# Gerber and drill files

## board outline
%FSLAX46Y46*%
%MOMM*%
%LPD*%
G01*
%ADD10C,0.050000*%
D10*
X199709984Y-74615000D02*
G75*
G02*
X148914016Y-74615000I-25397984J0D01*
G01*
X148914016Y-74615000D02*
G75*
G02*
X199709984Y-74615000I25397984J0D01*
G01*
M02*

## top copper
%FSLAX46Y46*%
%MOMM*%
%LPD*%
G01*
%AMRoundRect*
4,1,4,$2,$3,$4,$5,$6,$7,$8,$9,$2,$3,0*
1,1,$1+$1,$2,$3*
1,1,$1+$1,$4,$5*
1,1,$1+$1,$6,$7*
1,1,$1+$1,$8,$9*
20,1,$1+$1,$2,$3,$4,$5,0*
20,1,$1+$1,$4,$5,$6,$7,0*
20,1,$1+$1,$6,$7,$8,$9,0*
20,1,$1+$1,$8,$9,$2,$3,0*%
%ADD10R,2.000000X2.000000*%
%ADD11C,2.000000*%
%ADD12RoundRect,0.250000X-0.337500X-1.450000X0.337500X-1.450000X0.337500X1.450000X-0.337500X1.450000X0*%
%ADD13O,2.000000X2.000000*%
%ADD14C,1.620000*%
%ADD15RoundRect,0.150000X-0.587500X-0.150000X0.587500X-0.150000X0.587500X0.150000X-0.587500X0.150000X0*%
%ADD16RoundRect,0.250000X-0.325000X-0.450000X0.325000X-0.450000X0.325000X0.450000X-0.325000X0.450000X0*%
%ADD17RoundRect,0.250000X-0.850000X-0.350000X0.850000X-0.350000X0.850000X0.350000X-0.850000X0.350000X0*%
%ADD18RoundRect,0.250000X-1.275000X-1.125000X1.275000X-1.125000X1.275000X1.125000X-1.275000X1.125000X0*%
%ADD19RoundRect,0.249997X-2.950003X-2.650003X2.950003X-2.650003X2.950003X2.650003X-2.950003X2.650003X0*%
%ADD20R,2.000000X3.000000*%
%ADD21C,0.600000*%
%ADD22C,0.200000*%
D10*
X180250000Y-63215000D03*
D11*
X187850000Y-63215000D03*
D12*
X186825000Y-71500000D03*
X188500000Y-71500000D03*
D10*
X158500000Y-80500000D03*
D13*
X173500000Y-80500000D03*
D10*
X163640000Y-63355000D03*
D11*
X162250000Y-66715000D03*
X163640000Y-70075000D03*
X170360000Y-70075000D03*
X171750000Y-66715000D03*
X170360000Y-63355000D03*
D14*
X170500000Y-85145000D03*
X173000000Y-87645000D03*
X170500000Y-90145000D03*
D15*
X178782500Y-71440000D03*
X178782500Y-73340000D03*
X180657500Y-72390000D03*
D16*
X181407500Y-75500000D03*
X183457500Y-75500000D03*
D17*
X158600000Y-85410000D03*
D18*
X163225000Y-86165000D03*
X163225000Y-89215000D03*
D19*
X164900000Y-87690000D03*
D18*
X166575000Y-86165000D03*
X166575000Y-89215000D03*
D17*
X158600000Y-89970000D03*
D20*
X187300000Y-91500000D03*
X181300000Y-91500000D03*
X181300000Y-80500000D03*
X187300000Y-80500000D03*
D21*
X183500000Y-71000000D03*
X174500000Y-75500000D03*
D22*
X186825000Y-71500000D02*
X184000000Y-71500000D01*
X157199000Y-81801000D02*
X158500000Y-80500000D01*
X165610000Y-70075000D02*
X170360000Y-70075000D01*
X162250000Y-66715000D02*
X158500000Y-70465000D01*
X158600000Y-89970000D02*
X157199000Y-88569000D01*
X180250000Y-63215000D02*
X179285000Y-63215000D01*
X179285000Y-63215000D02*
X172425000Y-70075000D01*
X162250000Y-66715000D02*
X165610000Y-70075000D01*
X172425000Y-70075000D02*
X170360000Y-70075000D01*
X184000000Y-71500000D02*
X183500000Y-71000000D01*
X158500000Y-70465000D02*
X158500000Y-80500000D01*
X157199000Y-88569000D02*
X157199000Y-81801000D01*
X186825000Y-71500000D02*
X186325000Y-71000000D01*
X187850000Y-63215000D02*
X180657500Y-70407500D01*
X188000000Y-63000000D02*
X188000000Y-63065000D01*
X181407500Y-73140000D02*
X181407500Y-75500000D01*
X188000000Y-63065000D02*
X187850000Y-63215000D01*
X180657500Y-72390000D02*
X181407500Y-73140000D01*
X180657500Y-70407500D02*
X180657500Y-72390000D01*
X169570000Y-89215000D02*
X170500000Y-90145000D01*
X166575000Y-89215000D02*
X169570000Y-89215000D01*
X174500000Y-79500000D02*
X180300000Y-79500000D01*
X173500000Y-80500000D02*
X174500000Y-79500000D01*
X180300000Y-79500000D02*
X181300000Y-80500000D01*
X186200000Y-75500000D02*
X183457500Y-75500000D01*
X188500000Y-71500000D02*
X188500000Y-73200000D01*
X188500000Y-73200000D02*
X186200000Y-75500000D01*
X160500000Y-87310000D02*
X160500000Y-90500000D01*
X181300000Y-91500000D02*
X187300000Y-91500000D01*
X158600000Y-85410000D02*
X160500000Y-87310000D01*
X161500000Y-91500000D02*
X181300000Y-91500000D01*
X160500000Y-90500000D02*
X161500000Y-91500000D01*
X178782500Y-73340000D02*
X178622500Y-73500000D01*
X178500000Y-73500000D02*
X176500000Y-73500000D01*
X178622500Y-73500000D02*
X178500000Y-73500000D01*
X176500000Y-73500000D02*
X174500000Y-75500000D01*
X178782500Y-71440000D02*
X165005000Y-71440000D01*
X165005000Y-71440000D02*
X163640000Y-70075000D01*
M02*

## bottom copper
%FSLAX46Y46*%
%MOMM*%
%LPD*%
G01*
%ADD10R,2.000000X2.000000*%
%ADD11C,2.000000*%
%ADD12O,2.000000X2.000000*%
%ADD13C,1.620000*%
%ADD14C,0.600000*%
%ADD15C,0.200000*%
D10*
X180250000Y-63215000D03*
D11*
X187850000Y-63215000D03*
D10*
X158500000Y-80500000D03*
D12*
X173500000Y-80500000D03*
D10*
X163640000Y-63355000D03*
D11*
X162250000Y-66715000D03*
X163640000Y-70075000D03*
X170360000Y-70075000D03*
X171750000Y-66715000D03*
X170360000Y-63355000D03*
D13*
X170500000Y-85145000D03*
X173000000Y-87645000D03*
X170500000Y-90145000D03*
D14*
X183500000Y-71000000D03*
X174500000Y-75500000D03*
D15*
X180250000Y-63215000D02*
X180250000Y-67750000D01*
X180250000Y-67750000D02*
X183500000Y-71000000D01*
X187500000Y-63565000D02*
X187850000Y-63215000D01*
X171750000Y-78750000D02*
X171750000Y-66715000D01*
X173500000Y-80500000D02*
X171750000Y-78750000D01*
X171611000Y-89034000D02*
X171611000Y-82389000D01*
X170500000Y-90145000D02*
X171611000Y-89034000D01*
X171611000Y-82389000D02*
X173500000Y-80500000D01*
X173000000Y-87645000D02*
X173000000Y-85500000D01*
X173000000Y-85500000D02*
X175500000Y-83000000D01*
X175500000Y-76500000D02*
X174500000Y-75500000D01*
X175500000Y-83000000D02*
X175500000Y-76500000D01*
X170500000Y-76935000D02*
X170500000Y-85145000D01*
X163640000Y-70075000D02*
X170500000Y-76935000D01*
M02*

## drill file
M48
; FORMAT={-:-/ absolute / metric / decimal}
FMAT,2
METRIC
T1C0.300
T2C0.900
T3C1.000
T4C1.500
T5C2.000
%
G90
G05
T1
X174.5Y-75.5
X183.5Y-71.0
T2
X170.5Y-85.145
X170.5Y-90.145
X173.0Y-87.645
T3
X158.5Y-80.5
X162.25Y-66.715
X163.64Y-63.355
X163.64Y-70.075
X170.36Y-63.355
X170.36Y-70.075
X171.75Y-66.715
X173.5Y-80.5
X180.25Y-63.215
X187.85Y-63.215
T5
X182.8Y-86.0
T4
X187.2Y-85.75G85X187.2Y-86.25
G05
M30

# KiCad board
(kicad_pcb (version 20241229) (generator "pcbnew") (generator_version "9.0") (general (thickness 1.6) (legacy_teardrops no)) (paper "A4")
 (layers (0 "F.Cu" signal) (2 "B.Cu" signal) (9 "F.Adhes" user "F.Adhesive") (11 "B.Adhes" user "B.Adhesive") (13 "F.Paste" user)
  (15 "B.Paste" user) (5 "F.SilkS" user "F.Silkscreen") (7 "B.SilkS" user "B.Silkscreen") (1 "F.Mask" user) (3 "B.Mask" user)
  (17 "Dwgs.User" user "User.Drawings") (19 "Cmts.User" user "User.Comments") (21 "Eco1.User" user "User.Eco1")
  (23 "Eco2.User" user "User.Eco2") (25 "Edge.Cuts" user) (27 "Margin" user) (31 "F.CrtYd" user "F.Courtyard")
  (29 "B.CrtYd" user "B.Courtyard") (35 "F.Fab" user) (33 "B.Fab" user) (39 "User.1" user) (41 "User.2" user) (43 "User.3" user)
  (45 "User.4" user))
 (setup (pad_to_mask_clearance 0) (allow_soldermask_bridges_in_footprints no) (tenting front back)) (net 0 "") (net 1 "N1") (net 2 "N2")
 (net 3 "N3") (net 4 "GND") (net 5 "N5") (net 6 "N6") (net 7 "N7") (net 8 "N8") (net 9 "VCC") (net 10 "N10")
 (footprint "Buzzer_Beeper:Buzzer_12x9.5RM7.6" (layer "F.Cu") (at 180.25 63.215)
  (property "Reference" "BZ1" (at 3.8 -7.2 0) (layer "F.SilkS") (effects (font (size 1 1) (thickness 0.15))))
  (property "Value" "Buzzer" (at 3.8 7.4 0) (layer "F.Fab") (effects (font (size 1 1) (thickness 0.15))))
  (pad "1" thru_hole rect (at 0 0) (size 2 2) (drill 1) (layers "*.Cu" "*.Mask") (remove_unused_layers no) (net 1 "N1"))
  (pad "2" thru_hole circle (at 7.6 0) (size 2 2) (drill 1) (layers "*.Cu" "*.Mask") (remove_unused_layers no) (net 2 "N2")))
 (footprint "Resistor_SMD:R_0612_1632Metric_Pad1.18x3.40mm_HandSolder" (layer "F.Cu") (at 187.6625 71.5)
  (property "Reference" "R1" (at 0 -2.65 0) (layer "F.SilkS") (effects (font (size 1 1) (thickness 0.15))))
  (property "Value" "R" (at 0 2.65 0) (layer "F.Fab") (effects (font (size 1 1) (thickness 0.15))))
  (pad "1" smd roundrect (at -0.8375 0) (size 1.175 3.4) (layers "F.Cu" "F.Mask" "F.Paste") (roundrect_rratio 0.212766) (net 1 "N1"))
  (pad "2" smd roundrect (at 0.8375 0) (size 1.175 3.4) (layers "F.Cu" "F.Mask" "F.Paste") (roundrect_rratio 0.212766) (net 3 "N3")))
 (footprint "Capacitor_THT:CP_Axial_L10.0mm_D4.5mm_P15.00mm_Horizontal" (layer "F.Cu") (at 158.5 80.5)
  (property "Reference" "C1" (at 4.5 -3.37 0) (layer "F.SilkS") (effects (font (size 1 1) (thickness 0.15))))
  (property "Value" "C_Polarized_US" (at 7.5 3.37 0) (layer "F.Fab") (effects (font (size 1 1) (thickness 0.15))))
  (pad "1" thru_hole rect (at 0 0) (size 2 2) (drill 1) (layers "*.Cu" "*.Mask") (remove_unused_layers no) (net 1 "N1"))
  (pad "2" thru_hole oval (at 15 0) (size 2 2) (drill 1) (layers "*.Cu" "*.Mask") (remove_unused_layers no) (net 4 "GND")))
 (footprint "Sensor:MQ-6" (layer "F.Cu") (at 163.64 63.355)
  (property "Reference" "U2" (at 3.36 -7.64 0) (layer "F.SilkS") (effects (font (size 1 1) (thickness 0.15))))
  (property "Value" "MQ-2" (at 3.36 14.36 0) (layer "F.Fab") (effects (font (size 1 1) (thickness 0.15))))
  (pad "1" thru_hole rect (at 0 0) (size 2 2) (drill 1) (layers "*.Cu" "*.Mask") (remove_unused_layers no) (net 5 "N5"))
  (pad "2" thru_hole circle (at -1.39 3.36) (size 2 2) (drill 1) (layers "*.Cu" "*.Mask") (remove_unused_layers no) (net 1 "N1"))
  (pad "3" thru_hole circle (at 0 6.72 90) (size 2 2) (drill 1) (layers "*.Cu" "*.Mask") (remove_unused_layers no) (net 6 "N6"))
  (pad "4" thru_hole circle (at 6.72 6.72 180) (size 2 2) (drill 1) (layers "*.Cu" "*.Mask") (remove_unused_layers no) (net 1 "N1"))
  (pad "5" thru_hole circle (at 8.11 3.36) (size 2 2) (drill 1) (layers "*.Cu" "*.Mask") (remove_unused_layers no) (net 4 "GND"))
  (pad "6" thru_hole circle (at 6.72 0 270) (size 2 2) (drill 1) (layers "*.Cu" "*.Mask") (remove_unused_layers no) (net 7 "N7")))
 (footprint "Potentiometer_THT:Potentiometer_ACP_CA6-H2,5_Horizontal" (layer "F.Cu") (at 170.5 85.145)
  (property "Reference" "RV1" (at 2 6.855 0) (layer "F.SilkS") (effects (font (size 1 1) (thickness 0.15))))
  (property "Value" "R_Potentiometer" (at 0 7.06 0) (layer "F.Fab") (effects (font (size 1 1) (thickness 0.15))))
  (pad "1" thru_hole circle (at 0 0) (size 1.62 1.62) (drill 0.9) (layers "*.Cu" "*.Mask") (remove_unused_layers no) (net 6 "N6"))
  (pad "2" thru_hole circle (at 2.5 2.5) (size 1.62 1.62) (drill 0.9) (layers "*.Cu" "*.Mask") (remove_unused_layers no) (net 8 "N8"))
  (pad "3" thru_hole circle (at 0 5) (size 1.62 1.62) (drill 0.9) (layers "*.Cu" "*.Mask") (remove_unused_layers no) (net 4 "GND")))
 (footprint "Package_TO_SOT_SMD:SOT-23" (layer "F.Cu") (at 179.72 72.39)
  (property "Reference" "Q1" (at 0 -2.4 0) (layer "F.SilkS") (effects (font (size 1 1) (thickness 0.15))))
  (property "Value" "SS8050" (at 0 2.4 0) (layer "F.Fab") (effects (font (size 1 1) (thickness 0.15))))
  (pad "1" smd roundrect (at -0.9375 -0.95) (size 1.475 0.6) (layers "F.Cu" "F.Mask" "F.Paste") (roundrect_rratio 0.25) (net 6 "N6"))
  (pad "2" smd roundrect (at -0.9375 0.95) (size 1.475 0.6) (layers "F.Cu" "F.Mask" "F.Paste") (roundrect_rratio 0.25) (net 8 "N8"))
  (pad "3" smd roundrect (at 0.9375 0) (size 1.475 0.6) (layers "F.Cu" "F.Mask" "F.Paste") (roundrect_rratio 0.25) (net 2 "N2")))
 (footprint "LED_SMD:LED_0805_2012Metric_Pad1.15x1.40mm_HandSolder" (layer "F.Cu") (at 182.4325 75.5)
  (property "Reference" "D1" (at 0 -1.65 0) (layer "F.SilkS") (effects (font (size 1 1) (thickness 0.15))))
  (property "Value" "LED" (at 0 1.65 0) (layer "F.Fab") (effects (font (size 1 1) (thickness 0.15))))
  (pad "1" smd roundrect (at -1.025 0) (size 1.15 1.4) (layers "F.Cu" "F.Mask" "F.Paste") (roundrect_rratio 0.217391) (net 2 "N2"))
  (pad "2" smd roundrect (at 1.025 0) (size 1.15 1.4) (layers "F.Cu" "F.Mask" "F.Paste") (roundrect_rratio 0.217391) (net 3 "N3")))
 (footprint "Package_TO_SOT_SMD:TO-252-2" (layer "F.Cu") (at 163.64 87.69)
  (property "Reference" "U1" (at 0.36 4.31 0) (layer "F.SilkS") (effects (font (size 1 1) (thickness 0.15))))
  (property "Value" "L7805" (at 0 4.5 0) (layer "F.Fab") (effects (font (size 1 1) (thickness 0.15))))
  (pad "1" smd roundrect (at -5.04 -2.28) (size 2.2 1.2) (layers "F.Cu" "F.Mask" "F.Paste") (roundrect_rratio 0.208333) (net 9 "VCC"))
  (pad "2" smd roundrect (at -0.415 -1.525) (size 3.05 2.75) (layers "F.Cu" "F.Paste") (roundrect_rratio 0.090909) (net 4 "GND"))
  (pad "2" smd roundrect (at -0.415 1.525) (size 3.05 2.75) (layers "F.Cu" "F.Paste") (roundrect_rratio 0.090909) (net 4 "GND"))
  (pad "2" smd roundrect (at 1.26 0) (size 6.4 5.8) (layers "F.Cu" "F.Mask") (roundrect_rratio 0.043103) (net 4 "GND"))
  (pad "2" smd roundrect (at 2.935 -1.525) (size 3.05 2.75) (layers "F.Cu" "F.Paste") (roundrect_rratio 0.090909) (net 4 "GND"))
  (pad "2" smd roundrect (at 2.935 1.525) (size 3.05 2.75) (layers "F.Cu" "F.Paste") (roundrect_rratio 0.090909) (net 4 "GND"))
  (pad "3" smd roundrect (at -5.04 2.28) (size 2.2 1.2) (layers "F.Cu" "F.Mask" "F.Paste") (roundrect_rratio 0.208333) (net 1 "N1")))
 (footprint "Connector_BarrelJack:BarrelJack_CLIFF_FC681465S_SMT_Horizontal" (layer "F.Cu") (at 184.3 86 180)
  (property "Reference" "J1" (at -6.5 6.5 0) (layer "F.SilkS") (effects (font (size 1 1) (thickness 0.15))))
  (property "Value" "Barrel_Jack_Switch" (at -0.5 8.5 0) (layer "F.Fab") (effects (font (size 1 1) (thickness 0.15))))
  (pad "" np_thru_hole oval (at -2.9 0 270) (size 2 1.5) (drill oval 2 1.5) (layers "*.Cu" "*.Mask"))
  (pad "" np_thru_hole circle (at 1.5 0 270) (size 2 2) (drill 2) (layers "*.Cu" "*.Mask"))
  (pad "1" smd rect (at -3 -5.5 270) (size 3 2) (layers "F.Cu" "F.Mask" "F.Paste") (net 9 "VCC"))
  (pad "1" smd rect (at 3 -5.5 270) (size 3 2) (layers "F.Cu" "F.Mask" "F.Paste") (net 9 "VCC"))
  (pad "2" smd rect (at 3 5.5 270) (size 3 2) (layers "F.Cu" "F.Mask" "F.Paste") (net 4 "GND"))
  (pad "3" smd rect (at -3 5.5 270) (size 3 2) (layers "F.Cu" "F.Mask" "F.Paste") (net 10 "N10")))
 (gr_circle (center 174.312 74.615) (end 173.5 100) (stroke (width 0.05) (type default)) (fill no) (layer "Edge.Cuts"))
 (segment (start 186.825 71.5) (end 184 71.5) (width 0.2) (layer "F.Cu") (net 1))
 (segment (start 157.199 81.801) (end 158.5 80.5) (width 0.2) (layer "F.Cu") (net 1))
 (segment (start 165.61 70.075) (end 170.36 70.075) (width 0.2) (layer "F.Cu") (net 1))
 (segment (start 162.25 66.715) (end 158.5 70.465) (width 0.2) (layer "F.Cu") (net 1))
 (segment (start 158.6 89.97) (end 157.199 88.569) (width 0.2) (layer "F.Cu") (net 1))
 (segment (start 180.25 63.215) (end 179.285 63.215) (width 0.2) (layer "F.Cu") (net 1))
 (segment (start 179.285 63.215) (end 172.425 70.075) (width 0.2) (layer "F.Cu") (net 1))
 (segment (start 162.25 66.715) (end 165.61 70.075) (width 0.2) (layer "F.Cu") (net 1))
 (segment (start 172.425 70.075) (end 170.36 70.075) (width 0.2) (layer "F.Cu") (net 1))
 (segment (start 184 71.5) (end 183.5 71) (width 0.2) (layer "F.Cu") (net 1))
 (segment (start 158.5 70.465) (end 158.5 80.5) (width 0.2) (layer "F.Cu") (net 1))
 (segment (start 157.199 88.569) (end 157.199 81.801) (width 0.2) (layer "F.Cu") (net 1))
 (segment (start 186.825 71.5) (end 186.325 71) (width 0.2) (layer "F.Cu") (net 1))
 (via (at 183.5 71) (size 0.6) (drill 0.3) (layers "F.Cu" "B.Cu") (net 1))
 (segment (start 180.25 63.215) (end 180.25 67.75) (width 0.2) (layer "B.Cu") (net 1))
 (segment (start 180.25 67.75) (end 183.5 71) (width 0.2) (layer "B.Cu") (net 1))
 (segment (start 187.85 63.215) (end 180.6575 70.4075) (width 0.2) (layer "F.Cu") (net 2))
 (segment (start 188 63) (end 188 63.065) (width 0.2) (layer "F.Cu") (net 2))
 (segment (start 181.4075 73.14) (end 181.4075 75.5) (width 0.2) (layer "F.Cu") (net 2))
 (segment (start 188 63.065) (end 187.85 63.215) (width 0.2) (layer "F.Cu") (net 2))
 (segment (start 180.6575 72.39) (end 181.4075 73.14) (width 0.2) (layer "F.Cu") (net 2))
 (segment (start 180.6575 70.4075) (end 180.6575 72.39) (width 0.2) (layer "F.Cu") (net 2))
 (segment (start 187.5 63.565) (end 187.85 63.215) (width 0.2) (layer "B.Cu") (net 2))
 (segment (start 169.57 89.215) (end 170.5 90.145) (width 0.2) (layer "F.Cu") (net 4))
 (segment (start 166.575 89.215) (end 169.57 89.215) (width 0.2) (layer "F.Cu") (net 4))
 (segment (start 174.5 79.5) (end 180.3 79.5) (width 0.2) (layer "F.Cu") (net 4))
 (segment (start 173.5 80.5) (end 174.5 79.5) (width 0.2) (layer "F.Cu") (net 4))
 (segment (start 180.3 79.5) (end 181.3 80.5) (width 0.2) (layer "F.Cu") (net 4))
 (segment (start 171.75 78.75) (end 171.75 66.715) (width 0.2) (layer "B.Cu") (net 4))
 (segment (start 173.5 80.5) (end 171.75 78.75) (width 0.2) (layer "B.Cu") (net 4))
 (segment (start 171.611 89.034) (end 171.611 82.389) (width 0.2) (layer "B.Cu") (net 4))
 (segment (start 170.5 90.145) (end 171.611 89.034) (width 0.2) (layer "B.Cu") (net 4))
 (segment (start 171.611 82.389) (end 173.5 80.5) (width 0.2) (layer "B.Cu") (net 4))
 (segment (start 186.2 75.5) (end 183.4575 75.5) (width 0.2) (layer "F.Cu") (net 3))
 (segment (start 188.5 71.5) (end 188.5 73.2) (width 0.2) (layer "F.Cu") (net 3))
 (segment (start 188.5 73.2) (end 186.2 75.5) (width 0.2) (layer "F.Cu") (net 3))
 (segment (start 160.5 87.31) (end 160.5 90.5) (width 0.2) (layer "F.Cu") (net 9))
 (segment (start 181.3 91.5) (end 187.3 91.5) (width 0.2) (layer "F.Cu") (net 9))
 (segment (start 158.6 85.41) (end 160.5 87.31) (width 0.2) (layer "F.Cu") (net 9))
 (segment (start 161.5 91.5) (end 181.3 91.5) (width 0.2) (layer "F.Cu") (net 9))
 (segment (start 160.5 90.5) (end 161.5 91.5) (width 0.2) (layer "F.Cu") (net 9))
 (segment (start 178.7825 73.34) (end 178.6225 73.5) (width 0.2) (layer "F.Cu") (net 8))
 (segment (start 178.5 73.5) (end 176.5 73.5) (width 0.2) (layer "F.Cu") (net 8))
 (segment (start 178.6225 73.5) (end 178.5 73.5) (width 0.2) (layer "F.Cu") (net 8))
 (segment (start 176.5 73.5) (end 174.5 75.5) (width 0.2) (layer "F.Cu") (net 8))
 (via (at 174.5 75.5) (size 0.6) (drill 0.3) (layers "F.Cu" "B.Cu") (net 8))
 (segment (start 173 87.645) (end 173 85.5) (width 0.2) (layer "B.Cu") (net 8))
 (segment (start 173 85.5) (end 175.5 83) (width 0.2) (layer "B.Cu") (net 8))
 (segment (start 175.5 76.5) (end 174.5 75.5) (width 0.2) (layer "B.Cu") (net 8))
 (segment (start 175.5 83) (end 175.5 76.5) (width 0.2) (layer "B.Cu") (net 8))
 (segment (start 178.7825 71.44) (end 165.005 71.44) (width 0.2) (layer "F.Cu") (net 6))
 (segment (start 165.005 71.44) (end 163.64 70.075) (width 0.2) (layer "F.Cu") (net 6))
 (segment (start 170.5 76.935) (end 170.5 85.145) (width 0.2) (layer "B.Cu") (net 6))
 (segment (start 163.64 70.075) (end 170.5 76.935) (width 0.2) (layer "B.Cu") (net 6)))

